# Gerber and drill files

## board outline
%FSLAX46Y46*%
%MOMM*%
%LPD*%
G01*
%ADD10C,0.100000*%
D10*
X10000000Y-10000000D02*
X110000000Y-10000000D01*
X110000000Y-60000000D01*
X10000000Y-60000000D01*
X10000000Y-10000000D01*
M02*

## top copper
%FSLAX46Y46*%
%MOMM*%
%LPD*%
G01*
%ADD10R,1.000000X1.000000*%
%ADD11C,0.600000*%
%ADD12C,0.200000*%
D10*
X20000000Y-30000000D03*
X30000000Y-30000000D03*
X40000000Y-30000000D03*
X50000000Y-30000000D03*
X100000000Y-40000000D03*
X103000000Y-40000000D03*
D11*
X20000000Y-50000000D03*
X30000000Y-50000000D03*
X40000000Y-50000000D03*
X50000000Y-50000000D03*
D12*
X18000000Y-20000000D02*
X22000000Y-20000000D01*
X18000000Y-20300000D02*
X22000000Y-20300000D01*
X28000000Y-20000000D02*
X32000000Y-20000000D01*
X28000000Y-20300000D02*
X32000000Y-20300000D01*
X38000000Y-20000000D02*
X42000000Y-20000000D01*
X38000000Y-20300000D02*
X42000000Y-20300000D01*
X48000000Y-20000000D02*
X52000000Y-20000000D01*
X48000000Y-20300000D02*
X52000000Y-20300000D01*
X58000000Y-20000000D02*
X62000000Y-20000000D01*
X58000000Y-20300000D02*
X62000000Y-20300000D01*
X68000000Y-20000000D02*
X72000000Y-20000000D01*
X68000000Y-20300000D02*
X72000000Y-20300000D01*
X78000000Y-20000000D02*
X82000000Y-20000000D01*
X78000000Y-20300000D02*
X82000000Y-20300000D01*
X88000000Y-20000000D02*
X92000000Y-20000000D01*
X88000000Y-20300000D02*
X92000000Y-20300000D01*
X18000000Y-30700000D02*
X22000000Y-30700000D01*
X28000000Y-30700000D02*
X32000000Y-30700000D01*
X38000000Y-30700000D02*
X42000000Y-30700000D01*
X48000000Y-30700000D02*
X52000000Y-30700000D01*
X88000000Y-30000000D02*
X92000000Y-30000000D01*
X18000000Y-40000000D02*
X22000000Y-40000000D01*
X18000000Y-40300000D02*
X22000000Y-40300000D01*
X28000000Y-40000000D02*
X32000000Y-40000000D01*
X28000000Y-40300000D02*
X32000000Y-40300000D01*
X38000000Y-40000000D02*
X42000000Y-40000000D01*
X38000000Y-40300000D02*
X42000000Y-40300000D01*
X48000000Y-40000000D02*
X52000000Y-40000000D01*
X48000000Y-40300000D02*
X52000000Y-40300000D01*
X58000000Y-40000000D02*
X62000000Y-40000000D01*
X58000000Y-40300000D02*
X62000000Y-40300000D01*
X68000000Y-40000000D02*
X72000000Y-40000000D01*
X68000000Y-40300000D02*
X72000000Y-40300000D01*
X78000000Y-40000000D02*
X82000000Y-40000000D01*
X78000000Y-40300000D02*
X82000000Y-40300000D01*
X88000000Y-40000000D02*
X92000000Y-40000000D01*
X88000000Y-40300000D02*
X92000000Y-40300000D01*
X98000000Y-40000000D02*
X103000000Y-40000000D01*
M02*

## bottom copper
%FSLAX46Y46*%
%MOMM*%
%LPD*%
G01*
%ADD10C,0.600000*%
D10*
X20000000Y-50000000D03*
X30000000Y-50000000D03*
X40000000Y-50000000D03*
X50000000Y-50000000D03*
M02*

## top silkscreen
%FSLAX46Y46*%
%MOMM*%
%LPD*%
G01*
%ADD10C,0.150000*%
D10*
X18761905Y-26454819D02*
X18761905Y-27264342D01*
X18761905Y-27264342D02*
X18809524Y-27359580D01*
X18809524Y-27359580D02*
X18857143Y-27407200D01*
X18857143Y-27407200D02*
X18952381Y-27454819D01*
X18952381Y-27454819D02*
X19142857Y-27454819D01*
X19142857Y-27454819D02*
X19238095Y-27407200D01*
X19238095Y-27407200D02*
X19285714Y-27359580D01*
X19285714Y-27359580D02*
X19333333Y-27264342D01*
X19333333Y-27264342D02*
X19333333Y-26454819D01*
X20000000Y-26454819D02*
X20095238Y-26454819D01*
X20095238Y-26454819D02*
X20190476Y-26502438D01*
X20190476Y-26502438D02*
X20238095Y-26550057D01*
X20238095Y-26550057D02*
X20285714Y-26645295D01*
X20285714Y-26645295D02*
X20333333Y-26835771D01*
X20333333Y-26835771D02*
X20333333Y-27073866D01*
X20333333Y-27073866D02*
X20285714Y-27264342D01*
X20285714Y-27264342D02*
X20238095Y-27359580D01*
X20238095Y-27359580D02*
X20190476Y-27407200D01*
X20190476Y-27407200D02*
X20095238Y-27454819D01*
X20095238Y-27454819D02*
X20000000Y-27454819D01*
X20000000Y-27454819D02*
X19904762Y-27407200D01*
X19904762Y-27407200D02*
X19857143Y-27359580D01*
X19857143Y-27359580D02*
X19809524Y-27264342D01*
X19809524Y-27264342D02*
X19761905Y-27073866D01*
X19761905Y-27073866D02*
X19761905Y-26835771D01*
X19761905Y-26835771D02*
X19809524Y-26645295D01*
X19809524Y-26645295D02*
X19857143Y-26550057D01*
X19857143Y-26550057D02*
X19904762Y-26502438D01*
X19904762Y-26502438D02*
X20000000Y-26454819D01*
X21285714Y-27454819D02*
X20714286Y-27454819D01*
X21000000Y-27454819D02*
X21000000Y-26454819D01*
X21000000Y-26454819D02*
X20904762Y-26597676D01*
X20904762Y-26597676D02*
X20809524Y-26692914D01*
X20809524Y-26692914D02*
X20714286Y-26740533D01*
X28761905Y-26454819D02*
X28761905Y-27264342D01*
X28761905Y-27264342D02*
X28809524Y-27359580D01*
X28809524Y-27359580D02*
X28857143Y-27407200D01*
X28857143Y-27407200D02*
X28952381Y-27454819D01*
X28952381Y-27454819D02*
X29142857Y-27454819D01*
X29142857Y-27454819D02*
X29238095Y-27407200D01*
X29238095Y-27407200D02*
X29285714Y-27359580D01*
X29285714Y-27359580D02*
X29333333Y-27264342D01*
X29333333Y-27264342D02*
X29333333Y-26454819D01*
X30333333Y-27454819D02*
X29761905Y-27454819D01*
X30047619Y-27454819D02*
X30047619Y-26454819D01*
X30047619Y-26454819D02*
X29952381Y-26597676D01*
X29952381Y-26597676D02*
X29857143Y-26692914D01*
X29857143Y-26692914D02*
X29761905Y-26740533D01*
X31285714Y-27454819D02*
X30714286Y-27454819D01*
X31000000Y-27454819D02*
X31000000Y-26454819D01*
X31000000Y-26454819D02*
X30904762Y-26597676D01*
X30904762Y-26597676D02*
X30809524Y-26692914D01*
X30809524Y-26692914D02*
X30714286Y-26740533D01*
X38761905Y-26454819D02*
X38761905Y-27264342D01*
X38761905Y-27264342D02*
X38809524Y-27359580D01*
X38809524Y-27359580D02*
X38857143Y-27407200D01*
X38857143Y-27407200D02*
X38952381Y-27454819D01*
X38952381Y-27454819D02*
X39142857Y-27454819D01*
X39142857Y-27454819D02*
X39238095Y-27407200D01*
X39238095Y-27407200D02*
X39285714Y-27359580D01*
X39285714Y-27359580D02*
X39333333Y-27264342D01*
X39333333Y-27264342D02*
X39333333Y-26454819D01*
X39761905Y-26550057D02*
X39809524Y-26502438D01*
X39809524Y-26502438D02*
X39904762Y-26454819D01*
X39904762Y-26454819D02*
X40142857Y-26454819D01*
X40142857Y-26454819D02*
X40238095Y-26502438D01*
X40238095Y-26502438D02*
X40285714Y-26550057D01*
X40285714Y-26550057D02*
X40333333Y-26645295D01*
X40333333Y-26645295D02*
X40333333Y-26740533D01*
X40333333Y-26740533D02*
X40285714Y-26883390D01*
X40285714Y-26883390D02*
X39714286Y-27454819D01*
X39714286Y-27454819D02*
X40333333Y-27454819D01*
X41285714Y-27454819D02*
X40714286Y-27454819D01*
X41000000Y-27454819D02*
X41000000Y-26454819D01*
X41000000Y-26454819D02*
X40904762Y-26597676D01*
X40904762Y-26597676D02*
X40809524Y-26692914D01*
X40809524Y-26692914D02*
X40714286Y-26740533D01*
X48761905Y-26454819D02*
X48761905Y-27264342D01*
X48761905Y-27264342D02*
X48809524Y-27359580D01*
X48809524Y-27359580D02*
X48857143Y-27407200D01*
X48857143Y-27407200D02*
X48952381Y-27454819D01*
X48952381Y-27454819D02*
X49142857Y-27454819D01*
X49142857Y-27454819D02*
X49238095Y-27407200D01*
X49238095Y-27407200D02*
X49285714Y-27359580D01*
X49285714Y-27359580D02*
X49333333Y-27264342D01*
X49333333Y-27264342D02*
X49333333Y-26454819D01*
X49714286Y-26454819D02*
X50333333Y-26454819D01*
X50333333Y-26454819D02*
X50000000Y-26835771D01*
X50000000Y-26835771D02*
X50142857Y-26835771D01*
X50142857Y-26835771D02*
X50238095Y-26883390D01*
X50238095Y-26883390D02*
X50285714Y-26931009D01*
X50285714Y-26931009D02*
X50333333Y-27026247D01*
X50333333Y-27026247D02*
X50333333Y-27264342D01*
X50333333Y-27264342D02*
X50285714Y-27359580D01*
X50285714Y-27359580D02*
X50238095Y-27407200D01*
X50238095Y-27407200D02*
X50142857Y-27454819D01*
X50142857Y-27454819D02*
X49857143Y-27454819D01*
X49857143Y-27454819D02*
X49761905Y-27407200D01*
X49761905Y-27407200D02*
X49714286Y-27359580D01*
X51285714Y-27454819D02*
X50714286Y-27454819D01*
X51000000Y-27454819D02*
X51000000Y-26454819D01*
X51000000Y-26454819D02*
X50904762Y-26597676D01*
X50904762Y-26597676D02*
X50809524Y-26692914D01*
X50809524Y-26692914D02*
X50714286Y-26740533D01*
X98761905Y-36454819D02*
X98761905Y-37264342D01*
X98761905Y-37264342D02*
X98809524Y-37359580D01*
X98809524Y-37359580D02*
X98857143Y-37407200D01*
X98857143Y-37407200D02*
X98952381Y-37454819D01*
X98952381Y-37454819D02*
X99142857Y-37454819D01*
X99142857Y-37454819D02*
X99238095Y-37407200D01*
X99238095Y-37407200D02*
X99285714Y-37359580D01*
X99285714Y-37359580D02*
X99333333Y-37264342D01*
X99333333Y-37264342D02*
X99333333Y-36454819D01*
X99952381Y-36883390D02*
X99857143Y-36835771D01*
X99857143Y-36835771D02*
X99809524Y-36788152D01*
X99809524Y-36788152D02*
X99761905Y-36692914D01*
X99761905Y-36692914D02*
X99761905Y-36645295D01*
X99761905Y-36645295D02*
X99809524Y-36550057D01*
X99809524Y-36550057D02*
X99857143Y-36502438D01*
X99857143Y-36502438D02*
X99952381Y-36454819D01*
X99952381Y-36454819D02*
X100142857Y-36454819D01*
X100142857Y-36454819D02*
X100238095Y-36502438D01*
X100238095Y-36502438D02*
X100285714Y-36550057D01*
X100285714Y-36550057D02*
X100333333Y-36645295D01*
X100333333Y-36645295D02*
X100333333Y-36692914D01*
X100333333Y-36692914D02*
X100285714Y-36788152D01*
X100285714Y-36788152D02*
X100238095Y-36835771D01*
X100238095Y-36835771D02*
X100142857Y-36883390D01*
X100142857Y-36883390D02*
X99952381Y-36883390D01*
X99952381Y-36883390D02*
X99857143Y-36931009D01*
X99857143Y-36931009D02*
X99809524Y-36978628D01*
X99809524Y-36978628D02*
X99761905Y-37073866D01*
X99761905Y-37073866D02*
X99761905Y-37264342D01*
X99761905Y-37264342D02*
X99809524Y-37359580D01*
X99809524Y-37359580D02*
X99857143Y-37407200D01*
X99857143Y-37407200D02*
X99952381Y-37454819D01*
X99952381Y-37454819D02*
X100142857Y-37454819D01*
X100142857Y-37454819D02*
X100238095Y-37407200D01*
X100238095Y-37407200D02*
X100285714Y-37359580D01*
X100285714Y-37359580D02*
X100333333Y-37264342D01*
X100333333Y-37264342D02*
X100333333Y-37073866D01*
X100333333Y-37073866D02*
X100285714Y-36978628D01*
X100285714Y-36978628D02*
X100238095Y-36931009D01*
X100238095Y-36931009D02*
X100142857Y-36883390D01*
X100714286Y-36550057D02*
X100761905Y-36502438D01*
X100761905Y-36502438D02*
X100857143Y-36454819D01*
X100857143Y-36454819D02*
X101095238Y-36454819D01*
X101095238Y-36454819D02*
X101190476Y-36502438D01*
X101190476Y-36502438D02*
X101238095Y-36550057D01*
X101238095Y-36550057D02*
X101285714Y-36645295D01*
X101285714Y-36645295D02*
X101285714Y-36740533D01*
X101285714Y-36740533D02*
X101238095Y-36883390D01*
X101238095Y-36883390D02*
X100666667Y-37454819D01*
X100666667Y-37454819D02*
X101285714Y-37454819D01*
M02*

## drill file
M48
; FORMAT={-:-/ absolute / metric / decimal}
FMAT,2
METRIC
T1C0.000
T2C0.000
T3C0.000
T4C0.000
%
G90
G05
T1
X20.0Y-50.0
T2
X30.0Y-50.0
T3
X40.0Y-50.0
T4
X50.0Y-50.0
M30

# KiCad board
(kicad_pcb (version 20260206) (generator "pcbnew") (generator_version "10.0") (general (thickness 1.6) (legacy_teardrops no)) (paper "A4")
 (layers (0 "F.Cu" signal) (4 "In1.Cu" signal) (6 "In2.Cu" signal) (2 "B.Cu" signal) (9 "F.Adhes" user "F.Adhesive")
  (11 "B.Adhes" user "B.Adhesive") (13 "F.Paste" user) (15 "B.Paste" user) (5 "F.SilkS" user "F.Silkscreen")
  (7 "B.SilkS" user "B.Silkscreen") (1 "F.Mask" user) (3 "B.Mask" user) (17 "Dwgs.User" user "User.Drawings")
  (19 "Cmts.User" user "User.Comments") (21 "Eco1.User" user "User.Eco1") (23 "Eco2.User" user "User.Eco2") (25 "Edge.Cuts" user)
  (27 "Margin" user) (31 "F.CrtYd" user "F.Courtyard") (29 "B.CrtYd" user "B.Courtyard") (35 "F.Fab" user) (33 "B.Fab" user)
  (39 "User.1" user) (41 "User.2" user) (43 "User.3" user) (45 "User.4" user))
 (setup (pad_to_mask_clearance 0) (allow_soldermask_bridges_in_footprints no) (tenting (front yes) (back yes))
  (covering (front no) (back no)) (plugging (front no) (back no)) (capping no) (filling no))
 (segment (start 18 20) (end 22 20) (width 0.2) (layer "F.Cu") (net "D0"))
 (segment (start 18 20.3) (end 22 20.3) (width 0.2) (layer "F.Cu") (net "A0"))
 (segment (start 28 20) (end 32 20) (width 0.2) (layer "F.Cu") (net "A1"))
 (segment (start 28 20.3) (end 32 20.3) (width 0.2) (layer "F.Cu") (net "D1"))
 (segment (start 38 20) (end 42 20) (width 0.2) (layer "F.Cu") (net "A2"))
 (segment (start 38 20.3) (end 42 20.3) (width 0.2) (layer "F.Cu") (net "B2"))
 (segment (start 48 20) (end 52 20) (width 0.2) (layer "F.Cu") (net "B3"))
 (segment (start 48 20.3) (end 52 20.3) (width 0.2) (layer "F.Cu") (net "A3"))
 (segment (start 58 20) (end 62 20) (width 0.2) (layer "F.Cu") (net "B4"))
 (segment (start 58 20.3) (end 62 20.3) (width 0.2) (layer "F.Cu") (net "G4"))
 (segment (start 68 20) (end 72 20) (width 0.2) (layer "F.Cu") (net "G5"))
 (segment (start 68 20.3) (end 72 20.3) (width 0.2) (layer "F.Cu") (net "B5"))
 (segment (start 78 20) (end 82 20) (width 0.2) (layer "F.Cu") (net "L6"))
 (segment (start 78 20.3) (end 82 20.3) (width 0.2) (layer "F.Cu") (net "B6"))
 (segment (start 88 20) (end 92 20) (width 0.2) (layer "F.Cu") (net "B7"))
 (segment (start 88 20.3) (end 92 20.3) (width 0.2) (layer "F.Cu") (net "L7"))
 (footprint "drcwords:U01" (layer "F.Cu") (at 20 30)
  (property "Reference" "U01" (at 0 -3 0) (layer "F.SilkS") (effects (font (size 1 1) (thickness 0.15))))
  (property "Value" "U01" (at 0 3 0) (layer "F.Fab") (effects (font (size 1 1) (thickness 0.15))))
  (pad "1" smd rect (at 0 0) (size 1 1) (layers "F.Cu" "F.Mask" "F.Paste") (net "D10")))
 (segment (start 18 30.7) (end 22 30.7) (width 0.2) (layer "F.Cu") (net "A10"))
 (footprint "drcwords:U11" (layer "F.Cu") (at 30 30)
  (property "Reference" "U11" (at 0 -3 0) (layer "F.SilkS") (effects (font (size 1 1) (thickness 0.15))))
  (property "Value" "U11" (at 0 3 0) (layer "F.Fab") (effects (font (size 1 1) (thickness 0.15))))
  (pad "1" smd rect (at 0 0) (size 1 1) (layers "F.Cu" "F.Mask" "F.Paste") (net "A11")))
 (segment (start 28 30.7) (end 32 30.7) (width 0.2) (layer "F.Cu") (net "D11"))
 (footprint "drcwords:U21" (layer "F.Cu") (at 40 30)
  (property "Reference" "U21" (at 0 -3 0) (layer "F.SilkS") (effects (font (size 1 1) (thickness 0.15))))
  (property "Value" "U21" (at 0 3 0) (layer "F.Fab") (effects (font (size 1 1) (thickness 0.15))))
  (pad "1" smd rect (at 0 0) (size 1 1) (layers "F.Cu" "F.Mask" "F.Paste") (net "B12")))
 (segment (start 38 30.7) (end 42 30.7) (width 0.2) (layer "F.Cu") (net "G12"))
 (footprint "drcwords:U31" (layer "F.Cu") (at 50 30)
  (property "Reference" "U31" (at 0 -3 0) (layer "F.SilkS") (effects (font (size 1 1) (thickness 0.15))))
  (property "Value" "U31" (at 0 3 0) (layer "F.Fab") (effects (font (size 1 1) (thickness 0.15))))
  (pad "1" smd rect (at 0 0) (size 1 1) (layers "F.Cu" "F.Mask" "F.Paste") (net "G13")))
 (segment (start 48 30.7) (end 52 30.7) (width 0.2) (layer "F.Cu") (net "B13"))
 (segment (start 88 30) (end 92 30) (width 0.2) (layer "F.Cu") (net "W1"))
 (segment (start 18 40) (end 22 40) (width 0.2) (layer "F.Cu") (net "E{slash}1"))
 (segment (start 18 40.3) (end 22 40.3) (width 0.2) (layer "F.Cu") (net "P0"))
 (segment (start 28 40) (end 32 40) (width 0.2) (layer "F.Cu") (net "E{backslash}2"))
 (segment (start 28 40.3) (end 32 40.3) (width 0.2) (layer "F.Cu") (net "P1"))
 (segment (start 38 40) (end 42 40) (width 0.2) (layer "F.Cu") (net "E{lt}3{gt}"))
 (segment (start 38 40.3) (end 42 40.3) (width 0.2) (layer "F.Cu") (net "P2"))
 (segment (start 48 40) (end 52 40) (width 0.2) (layer "F.Cu") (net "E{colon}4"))
 (segment (start 48 40.3) (end 52 40.3) (width 0.2) (layer "F.Cu") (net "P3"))
 (segment (start 58 40) (end 62 40) (width 0.2) (layer "F.Cu") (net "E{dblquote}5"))
 (segment (start 58 40.3) (end 62 40.3) (width 0.2) (layer "F.Cu") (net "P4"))
 (segment (start 68 40) (end 72 40) (width 0.2) (layer "F.Cu") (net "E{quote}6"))
 (segment (start 68 40.3) (end 72 40.3) (width 0.2) (layer "F.Cu") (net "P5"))
 (segment (start 78 40) (end 82 40) (width 0.2) (layer "F.Cu") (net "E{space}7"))
 (segment (start 78 40.3) (end 82 40.3) (width 0.2) (layer "F.Cu") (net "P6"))
 (segment (start 88 40) (end 92 40) (width 0.2) (layer "F.Cu") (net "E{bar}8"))
 (segment (start 88 40.3) (end 92 40.3) (width 0.2) (layer "F.Cu") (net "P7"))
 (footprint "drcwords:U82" (layer "F.Cu") (at 100 40)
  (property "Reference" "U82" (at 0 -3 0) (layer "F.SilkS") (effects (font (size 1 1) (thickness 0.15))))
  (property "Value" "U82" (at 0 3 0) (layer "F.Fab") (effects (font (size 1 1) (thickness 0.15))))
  (pad "1" smd rect (at 0 0) (size 1 1) (layers "F.Cu" "F.Mask" "F.Paste") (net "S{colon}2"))
  (pad "2" smd rect (at 3 0) (size 1 1) (layers "F.Cu" "F.Mask" "F.Paste") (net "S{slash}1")))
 (segment (start 98 40) (end 103 40) (width 0.2) (layer "F.Cu") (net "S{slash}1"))
 (via (at 20 50) (size 0.6) (drill 0.00001) (layers "F.Cu" "B.Cu") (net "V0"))
 (via (at 30 50) (size 0.6) (drill 0.00004) (layers "F.Cu" "B.Cu") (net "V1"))
 (via (at 40 50) (size 0.6) (drill 0.00005) (layers "F.Cu" "B.Cu") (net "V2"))
 (via (at 50 50) (size 0.6) (drill 0.0001) (layers "F.Cu" "B.Cu") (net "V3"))
 (gr_rect (start 10 10) (end 110 60) (stroke (width 0.1) (type solid)) (fill no) (layer "Edge.Cuts")))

